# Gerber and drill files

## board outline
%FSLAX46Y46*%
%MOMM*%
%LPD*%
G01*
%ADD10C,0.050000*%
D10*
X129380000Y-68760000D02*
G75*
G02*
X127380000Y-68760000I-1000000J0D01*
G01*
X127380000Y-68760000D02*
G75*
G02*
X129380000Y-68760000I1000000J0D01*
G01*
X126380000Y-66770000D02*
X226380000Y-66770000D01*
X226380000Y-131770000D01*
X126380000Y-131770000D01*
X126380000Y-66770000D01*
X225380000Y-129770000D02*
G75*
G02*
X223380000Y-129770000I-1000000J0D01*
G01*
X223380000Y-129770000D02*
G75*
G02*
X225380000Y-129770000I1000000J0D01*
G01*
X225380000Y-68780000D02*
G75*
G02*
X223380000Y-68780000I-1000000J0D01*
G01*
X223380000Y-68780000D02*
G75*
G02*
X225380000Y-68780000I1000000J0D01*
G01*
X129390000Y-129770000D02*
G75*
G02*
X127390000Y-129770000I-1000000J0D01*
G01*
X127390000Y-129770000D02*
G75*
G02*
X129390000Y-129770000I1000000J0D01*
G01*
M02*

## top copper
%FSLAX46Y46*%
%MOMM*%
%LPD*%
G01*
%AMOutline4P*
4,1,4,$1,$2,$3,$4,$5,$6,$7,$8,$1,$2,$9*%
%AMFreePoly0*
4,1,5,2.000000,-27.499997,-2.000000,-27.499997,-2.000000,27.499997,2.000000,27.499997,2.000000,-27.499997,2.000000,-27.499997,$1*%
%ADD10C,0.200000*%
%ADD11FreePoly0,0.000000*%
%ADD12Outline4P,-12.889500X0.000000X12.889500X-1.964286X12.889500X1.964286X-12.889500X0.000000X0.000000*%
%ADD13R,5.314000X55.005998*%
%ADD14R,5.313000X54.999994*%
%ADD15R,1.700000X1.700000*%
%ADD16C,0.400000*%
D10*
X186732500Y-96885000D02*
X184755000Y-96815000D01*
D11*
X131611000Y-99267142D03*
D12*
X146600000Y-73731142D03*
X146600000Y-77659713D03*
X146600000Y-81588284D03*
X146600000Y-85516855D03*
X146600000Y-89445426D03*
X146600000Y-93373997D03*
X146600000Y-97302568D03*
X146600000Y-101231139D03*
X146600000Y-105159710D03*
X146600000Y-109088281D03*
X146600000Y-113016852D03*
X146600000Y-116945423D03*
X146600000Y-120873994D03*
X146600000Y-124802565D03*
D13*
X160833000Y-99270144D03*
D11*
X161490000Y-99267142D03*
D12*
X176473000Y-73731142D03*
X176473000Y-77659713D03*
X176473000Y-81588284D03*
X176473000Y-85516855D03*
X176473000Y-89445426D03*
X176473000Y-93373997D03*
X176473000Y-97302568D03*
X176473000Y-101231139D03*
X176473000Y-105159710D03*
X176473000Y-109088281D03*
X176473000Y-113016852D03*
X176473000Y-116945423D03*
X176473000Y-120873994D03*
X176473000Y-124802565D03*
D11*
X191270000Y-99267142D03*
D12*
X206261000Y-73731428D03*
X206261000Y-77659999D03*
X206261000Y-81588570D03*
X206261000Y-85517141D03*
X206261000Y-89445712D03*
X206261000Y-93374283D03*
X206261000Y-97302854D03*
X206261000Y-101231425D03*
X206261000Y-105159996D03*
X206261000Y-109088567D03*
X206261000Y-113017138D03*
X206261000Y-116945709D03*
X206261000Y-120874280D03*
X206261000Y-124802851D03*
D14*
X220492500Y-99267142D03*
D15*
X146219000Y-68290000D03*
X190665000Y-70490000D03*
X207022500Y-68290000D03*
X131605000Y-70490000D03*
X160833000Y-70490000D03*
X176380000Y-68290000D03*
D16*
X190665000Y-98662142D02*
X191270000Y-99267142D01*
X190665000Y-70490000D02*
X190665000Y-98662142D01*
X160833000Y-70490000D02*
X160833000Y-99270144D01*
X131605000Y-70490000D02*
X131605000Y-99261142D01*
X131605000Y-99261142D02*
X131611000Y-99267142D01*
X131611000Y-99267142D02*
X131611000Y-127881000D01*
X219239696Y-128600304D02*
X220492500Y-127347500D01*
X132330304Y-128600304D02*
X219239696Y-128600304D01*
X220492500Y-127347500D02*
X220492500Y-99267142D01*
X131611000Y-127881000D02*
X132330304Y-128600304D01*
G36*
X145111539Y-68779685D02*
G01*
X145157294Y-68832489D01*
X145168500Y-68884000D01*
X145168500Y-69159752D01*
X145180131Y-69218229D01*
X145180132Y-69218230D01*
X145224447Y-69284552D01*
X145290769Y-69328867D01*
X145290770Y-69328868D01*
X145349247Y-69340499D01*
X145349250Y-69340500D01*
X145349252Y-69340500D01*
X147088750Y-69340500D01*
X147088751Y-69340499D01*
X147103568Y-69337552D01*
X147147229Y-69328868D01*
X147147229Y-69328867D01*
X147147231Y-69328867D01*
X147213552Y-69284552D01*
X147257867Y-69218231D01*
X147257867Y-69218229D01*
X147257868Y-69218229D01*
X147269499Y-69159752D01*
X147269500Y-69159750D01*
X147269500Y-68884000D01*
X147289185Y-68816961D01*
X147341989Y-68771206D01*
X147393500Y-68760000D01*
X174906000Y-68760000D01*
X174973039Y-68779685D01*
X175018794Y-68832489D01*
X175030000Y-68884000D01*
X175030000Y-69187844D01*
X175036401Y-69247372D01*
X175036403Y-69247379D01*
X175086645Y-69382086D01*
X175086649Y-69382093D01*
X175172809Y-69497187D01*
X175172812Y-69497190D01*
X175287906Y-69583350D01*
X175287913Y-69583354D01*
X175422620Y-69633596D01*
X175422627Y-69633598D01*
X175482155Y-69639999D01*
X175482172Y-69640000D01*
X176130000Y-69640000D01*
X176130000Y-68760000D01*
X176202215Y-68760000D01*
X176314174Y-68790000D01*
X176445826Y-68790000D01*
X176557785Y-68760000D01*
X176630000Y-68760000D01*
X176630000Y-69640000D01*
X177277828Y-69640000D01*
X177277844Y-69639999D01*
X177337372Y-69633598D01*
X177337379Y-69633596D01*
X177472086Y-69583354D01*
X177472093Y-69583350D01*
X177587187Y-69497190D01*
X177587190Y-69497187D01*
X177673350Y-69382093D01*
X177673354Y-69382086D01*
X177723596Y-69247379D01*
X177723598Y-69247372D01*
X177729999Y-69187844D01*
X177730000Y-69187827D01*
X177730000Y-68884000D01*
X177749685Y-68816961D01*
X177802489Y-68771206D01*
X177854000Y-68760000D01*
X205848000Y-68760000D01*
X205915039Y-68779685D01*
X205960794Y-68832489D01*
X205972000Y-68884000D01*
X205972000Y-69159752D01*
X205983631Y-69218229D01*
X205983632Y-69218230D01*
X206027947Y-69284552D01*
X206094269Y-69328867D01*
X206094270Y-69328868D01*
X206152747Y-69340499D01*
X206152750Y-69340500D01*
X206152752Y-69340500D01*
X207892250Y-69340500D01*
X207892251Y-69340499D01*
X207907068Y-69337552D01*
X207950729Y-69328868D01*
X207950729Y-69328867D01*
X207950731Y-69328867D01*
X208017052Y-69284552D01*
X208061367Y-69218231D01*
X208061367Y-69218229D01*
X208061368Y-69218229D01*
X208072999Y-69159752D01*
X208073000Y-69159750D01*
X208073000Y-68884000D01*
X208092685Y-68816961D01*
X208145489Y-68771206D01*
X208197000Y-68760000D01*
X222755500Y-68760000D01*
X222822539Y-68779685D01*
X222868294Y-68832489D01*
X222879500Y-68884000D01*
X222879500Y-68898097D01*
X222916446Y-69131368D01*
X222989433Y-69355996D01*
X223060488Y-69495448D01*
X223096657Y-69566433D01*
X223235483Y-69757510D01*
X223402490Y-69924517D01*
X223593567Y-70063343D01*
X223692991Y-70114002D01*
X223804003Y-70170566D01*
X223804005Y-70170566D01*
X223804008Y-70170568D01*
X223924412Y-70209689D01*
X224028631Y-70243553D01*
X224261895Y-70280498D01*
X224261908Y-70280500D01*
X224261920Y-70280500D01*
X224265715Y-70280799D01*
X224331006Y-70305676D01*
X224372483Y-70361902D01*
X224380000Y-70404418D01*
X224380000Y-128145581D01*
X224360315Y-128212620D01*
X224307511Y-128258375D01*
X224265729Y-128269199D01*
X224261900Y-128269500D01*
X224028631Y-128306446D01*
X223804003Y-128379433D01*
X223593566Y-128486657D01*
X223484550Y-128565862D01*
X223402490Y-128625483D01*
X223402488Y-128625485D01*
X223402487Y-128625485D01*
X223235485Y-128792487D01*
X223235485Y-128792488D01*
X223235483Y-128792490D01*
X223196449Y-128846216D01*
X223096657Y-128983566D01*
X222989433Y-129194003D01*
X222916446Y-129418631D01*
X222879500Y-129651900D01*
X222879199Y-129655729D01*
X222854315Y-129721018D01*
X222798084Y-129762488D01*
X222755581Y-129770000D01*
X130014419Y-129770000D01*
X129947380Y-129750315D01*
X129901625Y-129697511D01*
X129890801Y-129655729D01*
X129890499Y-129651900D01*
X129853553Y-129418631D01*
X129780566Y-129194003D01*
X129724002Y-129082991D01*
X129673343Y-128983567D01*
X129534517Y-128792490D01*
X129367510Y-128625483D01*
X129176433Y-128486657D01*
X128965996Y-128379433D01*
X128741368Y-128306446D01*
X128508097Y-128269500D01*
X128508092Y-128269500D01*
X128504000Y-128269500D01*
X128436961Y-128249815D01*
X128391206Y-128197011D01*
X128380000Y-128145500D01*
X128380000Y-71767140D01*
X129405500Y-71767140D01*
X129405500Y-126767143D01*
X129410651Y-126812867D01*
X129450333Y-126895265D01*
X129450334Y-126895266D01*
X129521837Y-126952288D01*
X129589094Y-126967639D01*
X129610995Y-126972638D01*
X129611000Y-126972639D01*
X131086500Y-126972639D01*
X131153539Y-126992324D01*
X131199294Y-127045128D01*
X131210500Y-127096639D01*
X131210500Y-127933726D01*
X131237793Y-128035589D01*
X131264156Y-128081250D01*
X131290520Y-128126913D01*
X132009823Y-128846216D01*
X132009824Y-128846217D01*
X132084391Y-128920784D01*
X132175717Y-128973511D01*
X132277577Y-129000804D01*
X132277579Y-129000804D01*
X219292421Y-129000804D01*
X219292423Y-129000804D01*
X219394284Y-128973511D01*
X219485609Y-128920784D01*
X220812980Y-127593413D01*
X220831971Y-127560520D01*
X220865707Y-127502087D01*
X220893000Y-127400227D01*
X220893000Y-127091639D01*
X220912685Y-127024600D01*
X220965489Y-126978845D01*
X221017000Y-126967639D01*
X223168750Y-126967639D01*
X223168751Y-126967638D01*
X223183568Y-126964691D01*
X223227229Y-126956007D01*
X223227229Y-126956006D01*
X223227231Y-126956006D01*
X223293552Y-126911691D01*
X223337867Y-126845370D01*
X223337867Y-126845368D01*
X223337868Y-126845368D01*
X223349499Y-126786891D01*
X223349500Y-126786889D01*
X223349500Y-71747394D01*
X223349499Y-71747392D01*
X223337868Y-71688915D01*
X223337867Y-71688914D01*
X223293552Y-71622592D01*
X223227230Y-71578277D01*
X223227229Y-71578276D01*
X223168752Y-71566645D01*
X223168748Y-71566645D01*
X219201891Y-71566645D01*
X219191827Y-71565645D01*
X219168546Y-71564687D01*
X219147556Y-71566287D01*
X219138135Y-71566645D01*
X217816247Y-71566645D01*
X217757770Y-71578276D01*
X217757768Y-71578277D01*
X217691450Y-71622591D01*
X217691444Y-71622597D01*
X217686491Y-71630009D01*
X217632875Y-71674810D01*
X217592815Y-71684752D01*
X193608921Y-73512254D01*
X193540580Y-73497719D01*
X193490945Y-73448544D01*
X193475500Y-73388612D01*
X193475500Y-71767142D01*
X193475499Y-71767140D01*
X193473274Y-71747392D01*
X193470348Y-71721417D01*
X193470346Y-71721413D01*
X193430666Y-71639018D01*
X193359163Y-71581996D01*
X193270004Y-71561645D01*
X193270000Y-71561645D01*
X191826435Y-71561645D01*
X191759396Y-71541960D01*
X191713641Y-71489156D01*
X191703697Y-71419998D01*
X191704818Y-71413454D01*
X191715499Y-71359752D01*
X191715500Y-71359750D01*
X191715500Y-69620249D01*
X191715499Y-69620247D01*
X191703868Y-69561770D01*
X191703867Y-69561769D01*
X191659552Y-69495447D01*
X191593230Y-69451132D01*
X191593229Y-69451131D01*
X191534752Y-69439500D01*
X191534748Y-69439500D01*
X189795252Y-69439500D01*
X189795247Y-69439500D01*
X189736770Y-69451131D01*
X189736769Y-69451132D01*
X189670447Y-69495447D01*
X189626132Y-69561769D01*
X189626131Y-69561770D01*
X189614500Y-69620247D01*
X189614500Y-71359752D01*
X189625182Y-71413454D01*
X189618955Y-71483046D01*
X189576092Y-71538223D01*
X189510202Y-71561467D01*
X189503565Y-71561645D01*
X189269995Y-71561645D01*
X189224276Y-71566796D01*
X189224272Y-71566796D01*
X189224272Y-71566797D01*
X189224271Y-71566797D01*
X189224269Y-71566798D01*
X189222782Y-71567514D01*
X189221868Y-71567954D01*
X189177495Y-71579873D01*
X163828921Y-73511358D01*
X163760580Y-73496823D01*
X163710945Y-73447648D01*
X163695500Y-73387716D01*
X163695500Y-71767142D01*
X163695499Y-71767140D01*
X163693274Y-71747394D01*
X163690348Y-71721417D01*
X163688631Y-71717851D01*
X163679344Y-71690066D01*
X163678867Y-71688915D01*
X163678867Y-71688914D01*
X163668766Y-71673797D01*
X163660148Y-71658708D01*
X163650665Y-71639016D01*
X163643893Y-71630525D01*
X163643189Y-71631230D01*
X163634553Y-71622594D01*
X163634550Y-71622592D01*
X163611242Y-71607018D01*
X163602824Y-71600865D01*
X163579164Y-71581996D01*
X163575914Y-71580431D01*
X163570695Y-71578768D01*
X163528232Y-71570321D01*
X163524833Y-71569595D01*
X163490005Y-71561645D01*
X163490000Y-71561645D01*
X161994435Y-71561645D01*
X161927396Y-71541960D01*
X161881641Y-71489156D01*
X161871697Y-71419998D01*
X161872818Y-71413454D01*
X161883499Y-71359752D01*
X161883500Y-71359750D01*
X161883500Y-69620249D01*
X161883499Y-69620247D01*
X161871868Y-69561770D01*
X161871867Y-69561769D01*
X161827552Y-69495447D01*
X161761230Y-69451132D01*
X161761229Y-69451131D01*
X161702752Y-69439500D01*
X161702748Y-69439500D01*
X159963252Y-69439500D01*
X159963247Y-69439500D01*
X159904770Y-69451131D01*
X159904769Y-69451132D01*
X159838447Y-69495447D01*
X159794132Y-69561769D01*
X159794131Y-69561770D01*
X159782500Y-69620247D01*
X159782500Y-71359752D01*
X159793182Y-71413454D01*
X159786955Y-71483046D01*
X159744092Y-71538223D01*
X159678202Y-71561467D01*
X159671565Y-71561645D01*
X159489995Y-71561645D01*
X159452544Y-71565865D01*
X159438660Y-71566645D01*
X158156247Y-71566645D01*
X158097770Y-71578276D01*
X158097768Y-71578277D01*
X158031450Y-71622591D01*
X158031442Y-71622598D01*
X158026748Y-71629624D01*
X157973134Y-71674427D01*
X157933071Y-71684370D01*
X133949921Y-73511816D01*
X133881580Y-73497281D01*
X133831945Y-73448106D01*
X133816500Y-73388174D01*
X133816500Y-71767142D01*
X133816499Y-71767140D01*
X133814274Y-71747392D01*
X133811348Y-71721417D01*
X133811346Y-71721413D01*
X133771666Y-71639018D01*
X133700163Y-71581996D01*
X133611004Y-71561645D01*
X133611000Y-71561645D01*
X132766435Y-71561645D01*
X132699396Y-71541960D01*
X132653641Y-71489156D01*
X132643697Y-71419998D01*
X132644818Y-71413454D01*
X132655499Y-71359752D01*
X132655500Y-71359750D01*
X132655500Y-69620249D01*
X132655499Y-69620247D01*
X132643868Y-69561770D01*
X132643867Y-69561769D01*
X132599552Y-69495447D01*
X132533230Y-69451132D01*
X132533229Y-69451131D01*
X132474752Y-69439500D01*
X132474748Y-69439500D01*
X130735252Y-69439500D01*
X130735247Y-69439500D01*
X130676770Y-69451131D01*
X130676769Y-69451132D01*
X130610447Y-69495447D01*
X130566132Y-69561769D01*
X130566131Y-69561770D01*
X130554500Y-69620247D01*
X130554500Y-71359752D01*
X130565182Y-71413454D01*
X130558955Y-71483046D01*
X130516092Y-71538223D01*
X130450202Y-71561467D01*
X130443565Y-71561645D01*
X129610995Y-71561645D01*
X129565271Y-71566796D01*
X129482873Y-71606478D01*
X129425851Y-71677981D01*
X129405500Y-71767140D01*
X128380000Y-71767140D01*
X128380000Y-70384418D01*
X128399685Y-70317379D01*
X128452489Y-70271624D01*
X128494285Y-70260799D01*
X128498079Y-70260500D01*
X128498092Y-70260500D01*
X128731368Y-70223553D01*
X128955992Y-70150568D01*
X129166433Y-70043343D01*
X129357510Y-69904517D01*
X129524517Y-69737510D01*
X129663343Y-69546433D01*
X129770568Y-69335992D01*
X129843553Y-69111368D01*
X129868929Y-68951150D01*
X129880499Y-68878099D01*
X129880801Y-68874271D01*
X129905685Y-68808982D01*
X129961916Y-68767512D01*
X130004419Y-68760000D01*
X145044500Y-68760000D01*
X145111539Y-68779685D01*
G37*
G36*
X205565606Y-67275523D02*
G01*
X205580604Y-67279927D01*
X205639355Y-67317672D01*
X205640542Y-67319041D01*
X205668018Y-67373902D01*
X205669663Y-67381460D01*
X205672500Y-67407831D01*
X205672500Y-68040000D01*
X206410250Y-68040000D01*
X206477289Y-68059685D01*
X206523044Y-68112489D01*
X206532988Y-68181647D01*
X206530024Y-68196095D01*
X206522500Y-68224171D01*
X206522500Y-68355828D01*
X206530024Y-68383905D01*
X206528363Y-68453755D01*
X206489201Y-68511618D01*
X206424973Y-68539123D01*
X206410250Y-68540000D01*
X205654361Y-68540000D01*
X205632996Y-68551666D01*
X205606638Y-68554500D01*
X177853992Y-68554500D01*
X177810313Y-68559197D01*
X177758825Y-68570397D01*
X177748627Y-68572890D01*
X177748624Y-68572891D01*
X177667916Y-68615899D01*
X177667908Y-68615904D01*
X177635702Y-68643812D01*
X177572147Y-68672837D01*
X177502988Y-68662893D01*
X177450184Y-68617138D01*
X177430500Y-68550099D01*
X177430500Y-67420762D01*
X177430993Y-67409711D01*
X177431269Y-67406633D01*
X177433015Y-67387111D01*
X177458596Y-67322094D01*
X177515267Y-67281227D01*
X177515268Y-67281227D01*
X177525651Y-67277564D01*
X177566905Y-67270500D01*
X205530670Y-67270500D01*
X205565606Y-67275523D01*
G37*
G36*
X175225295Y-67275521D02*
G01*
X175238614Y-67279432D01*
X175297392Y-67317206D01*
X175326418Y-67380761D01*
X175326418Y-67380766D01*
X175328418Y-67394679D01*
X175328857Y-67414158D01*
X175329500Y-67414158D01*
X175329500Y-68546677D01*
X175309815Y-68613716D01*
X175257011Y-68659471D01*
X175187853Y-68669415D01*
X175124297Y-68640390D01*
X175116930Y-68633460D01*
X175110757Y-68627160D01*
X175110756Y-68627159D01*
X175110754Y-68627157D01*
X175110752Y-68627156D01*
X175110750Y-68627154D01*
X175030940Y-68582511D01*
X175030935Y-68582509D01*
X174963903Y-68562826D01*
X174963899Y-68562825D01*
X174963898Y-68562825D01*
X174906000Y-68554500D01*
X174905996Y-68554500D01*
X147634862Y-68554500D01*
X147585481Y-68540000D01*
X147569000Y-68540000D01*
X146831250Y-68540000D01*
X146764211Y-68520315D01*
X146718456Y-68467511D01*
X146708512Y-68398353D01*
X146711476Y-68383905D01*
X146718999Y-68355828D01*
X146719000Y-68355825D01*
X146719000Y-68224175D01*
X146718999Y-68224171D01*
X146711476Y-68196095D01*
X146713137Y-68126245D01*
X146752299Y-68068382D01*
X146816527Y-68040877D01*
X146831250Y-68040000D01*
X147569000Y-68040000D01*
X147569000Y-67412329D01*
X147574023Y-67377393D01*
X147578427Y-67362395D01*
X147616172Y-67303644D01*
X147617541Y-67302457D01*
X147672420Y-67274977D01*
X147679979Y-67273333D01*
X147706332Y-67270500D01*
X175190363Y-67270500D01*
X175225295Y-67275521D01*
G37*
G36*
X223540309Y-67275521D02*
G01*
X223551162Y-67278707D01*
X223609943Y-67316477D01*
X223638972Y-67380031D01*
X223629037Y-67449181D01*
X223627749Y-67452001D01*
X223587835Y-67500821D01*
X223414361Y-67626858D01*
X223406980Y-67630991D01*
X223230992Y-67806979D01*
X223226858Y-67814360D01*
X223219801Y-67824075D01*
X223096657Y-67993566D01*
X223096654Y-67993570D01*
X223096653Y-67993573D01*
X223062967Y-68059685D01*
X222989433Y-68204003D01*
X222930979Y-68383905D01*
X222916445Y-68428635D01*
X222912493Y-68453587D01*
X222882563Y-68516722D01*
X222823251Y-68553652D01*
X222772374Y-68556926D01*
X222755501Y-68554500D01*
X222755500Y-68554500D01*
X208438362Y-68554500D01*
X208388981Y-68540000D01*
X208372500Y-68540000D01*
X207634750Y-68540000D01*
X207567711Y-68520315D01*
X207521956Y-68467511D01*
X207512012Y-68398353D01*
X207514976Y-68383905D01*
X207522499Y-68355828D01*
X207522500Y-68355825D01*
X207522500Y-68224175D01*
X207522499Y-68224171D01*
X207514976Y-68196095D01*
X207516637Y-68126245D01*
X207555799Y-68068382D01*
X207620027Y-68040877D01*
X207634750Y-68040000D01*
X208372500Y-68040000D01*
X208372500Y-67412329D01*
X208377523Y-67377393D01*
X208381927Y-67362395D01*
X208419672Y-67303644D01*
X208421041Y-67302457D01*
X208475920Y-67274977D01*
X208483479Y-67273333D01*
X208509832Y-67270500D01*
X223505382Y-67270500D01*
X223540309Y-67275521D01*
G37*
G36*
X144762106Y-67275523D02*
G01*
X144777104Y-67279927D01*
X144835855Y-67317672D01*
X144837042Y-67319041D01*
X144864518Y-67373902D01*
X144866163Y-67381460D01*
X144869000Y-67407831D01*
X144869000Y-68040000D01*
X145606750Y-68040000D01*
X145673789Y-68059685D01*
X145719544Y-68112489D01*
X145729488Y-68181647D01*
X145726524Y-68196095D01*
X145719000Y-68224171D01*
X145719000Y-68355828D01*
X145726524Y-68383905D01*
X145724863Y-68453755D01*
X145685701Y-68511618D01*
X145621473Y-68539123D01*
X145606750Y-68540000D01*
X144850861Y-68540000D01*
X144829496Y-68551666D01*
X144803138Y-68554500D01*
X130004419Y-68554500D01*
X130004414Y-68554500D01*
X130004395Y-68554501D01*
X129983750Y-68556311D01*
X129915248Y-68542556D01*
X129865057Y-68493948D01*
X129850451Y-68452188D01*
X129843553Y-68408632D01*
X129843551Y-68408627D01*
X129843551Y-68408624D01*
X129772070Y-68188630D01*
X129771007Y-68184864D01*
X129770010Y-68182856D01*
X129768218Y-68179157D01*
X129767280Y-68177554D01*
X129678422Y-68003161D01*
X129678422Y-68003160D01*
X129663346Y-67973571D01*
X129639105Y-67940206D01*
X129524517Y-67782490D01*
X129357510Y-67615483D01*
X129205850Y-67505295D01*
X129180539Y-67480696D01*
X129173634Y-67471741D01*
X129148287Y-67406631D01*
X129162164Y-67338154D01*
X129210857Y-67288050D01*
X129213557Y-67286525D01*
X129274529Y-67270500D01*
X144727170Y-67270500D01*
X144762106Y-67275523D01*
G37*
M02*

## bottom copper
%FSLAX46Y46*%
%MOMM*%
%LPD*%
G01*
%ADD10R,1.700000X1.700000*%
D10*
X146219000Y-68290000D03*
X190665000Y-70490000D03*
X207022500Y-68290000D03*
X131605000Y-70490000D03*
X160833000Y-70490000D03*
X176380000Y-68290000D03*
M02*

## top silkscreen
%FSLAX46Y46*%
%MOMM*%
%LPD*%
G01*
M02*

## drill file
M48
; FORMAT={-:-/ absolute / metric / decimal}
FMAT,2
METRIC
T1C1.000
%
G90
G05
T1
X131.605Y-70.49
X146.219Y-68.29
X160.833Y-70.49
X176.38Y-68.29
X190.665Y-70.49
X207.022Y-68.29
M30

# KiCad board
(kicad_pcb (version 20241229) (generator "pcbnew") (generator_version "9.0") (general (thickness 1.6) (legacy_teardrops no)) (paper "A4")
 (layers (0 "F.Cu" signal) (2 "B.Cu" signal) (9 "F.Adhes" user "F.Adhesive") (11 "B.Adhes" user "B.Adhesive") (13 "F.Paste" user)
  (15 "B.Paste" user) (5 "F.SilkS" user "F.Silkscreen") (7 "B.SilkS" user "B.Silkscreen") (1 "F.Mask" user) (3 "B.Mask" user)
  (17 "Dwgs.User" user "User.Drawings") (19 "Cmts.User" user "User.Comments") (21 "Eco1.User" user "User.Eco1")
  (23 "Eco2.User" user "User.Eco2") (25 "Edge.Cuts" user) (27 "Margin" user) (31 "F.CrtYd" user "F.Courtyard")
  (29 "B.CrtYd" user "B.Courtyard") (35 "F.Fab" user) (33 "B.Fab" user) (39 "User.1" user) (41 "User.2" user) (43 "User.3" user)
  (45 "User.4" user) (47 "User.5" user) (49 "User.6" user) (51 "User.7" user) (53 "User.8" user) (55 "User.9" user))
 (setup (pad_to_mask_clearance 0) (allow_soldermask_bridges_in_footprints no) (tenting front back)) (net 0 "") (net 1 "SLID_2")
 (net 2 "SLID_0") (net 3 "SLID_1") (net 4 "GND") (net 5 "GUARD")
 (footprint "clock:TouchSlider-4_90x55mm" (layer "F.Cu") (at 176.332 99.267142)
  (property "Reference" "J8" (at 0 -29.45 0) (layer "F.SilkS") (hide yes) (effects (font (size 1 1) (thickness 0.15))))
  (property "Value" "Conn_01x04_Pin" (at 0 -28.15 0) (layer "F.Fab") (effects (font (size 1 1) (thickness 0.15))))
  (pad "1" smd custom (at -44.721 0) (size 4 54.999994) (layers "F.Cu") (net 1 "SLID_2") (thermal_bridge_angle 45)
   (options (clearance outline) (anchor rect)) (primitives))
  (pad "2" smd trapezoid (at -29.732 -25.536) (size 25.779 1.964285) (rect_delta -1.964285 0) (layers "F.Cu" "F.Paste") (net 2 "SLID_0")
   (thermal_bridge_angle 45))
  (pad "2" smd trapezoid (at -29.732 -21.607429) (size 25.779 1.964285) (rect_delta -1.964285 0) (layers "F.Cu" "F.Paste") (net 2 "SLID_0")
   (thermal_bridge_angle 45))
  (pad "2" smd trapezoid (at -29.732 -17.678858) (size 25.779 1.964285) (rect_delta -1.964285 0) (layers "F.Cu" "F.Paste") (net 2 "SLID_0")
   (thermal_bridge_angle 45))
  (pad "2" smd trapezoid (at -29.732 -13.750287) (size 25.779 1.964285) (rect_delta -1.964285 0) (layers "F.Cu" "F.Paste") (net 2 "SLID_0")
   (thermal_bridge_angle 45))
  (pad "2" smd trapezoid (at -29.732 -9.821716) (size 25.779 1.964285) (rect_delta -1.964285 0) (layers "F.Cu" "F.Paste") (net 2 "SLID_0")
   (thermal_bridge_angle 45))
  (pad "2" smd trapezoid (at -29.732 -5.893145) (size 25.779 1.964285) (rect_delta -1.964285 0) (layers "F.Cu" "F.Paste") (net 2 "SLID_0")
   (thermal_bridge_angle 45))
  (pad "2" smd trapezoid (at -29.732 -1.964574) (size 25.779 1.964285) (rect_delta -1.964285 0) (layers "F.Cu" "F.Paste") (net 2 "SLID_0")
   (thermal_bridge_angle 45))
  (pad "2" smd trapezoid (at -29.732 1.963997) (size 25.779 1.964285) (rect_delta -1.964285 0) (layers "F.Cu" "F.Paste") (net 2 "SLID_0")
   (thermal_bridge_angle 45))
  (pad "2" smd trapezoid (at -29.732 5.892568) (size 25.779 1.964285) (rect_delta -1.964285 0) (layers "F.Cu" "F.Paste") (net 2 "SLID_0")
   (thermal_bridge_angle 45))
  (pad "2" smd trapezoid (at -29.732 9.821139) (size 25.779 1.964285) (rect_delta -1.964285 0) (layers "F.Cu" "F.Paste") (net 2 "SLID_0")
   (thermal_bridge_angle 45))
  (pad "2" smd trapezoid (at -29.732 13.74971) (size 25.779 1.964285) (rect_delta -1.964285 0) (layers "F.Cu" "F.Paste") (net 2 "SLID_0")
   (thermal_bridge_angle 45))
  (pad "2" smd trapezoid (at -29.732 17.678281) (size 25.779 1.964285) (rect_delta -1.964285 0) (layers "F.Cu" "F.Paste") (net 2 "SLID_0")
   (thermal_bridge_angle 45))
  (pad "2" smd trapezoid (at -29.732 21.606852) (size 25.779 1.964285) (rect_delta -1.964285 0) (layers "F.Cu" "F.Paste") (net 2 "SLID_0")
   (thermal_bridge_angle 45))
  (pad "2" smd trapezoid (at -29.732 25.535423) (size 25.779 1.964285) (rect_delta -1.964285 0) (layers "F.Cu" "F.Paste") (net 2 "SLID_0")
   (thermal_bridge_angle 45))
  (pad "2" smd rect (at -15.499 0.003002) (size 5.314 55.005998) (layers "F.Cu") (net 2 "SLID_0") (thermal_bridge_angle 45))
  (pad "2" smd custom (at -14.842 0) (size 4 54.999994) (layers "F.Cu") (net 2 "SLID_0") (thermal_bridge_angle 45)
   (options (clearance outline) (anchor rect)) (primitives))
  (pad "3" smd trapezoid (at 0.141 -25.536) (size 25.779 1.964285) (rect_delta -1.964285 0) (layers "F.Cu" "F.Paste") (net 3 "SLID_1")
   (thermal_bridge_angle 45))
  (pad "3" smd trapezoid (at 0.141 -21.607429) (size 25.779 1.964285) (rect_delta -1.964285 0) (layers "F.Cu" "F.Paste") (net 3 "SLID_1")
   (thermal_bridge_angle 45))
  (pad "3" smd trapezoid (at 0.141 -17.678858) (size 25.779 1.964285) (rect_delta -1.964285 0) (layers "F.Cu" "F.Paste") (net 3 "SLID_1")
   (thermal_bridge_angle 45))
  (pad "3" smd trapezoid (at 0.141 -13.750287) (size 25.779 1.964285) (rect_delta -1.964285 0) (layers "F.Cu" "F.Paste") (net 3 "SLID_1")
   (thermal_bridge_angle 45))
  (pad "3" smd trapezoid (at 0.141 -9.821716) (size 25.779 1.964285) (rect_delta -1.964285 0) (layers "F.Cu" "F.Paste") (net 3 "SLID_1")
   (thermal_bridge_angle 45))
  (pad "3" smd trapezoid (at 0.141 -5.893145) (size 25.779 1.964285) (rect_delta -1.964285 0) (layers "F.Cu" "F.Paste") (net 3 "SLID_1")
   (thermal_bridge_angle 45))
  (pad "3" smd trapezoid (at 0.141 -1.964574) (size 25.779 1.964285) (rect_delta -1.964285 0) (layers "F.Cu" "F.Paste") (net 3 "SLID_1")
   (thermal_bridge_angle 45))
  (pad "3" smd trapezoid (at 0.141 1.963997) (size 25.779 1.964285) (rect_delta -1.964285 0) (layers "F.Cu" "F.Paste") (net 3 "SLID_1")
   (thermal_bridge_angle 45))
  (pad "3" smd trapezoid (at 0.141 5.892568) (size 25.779 1.964285) (rect_delta -1.964285 0) (layers "F.Cu" "F.Paste") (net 3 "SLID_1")
   (thermal_bridge_angle 45))
  (pad "3" smd trapezoid (at 0.141 9.821139) (size 25.779 1.964285) (rect_delta -1.964285 0) (layers "F.Cu" "F.Paste") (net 3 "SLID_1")
   (thermal_bridge_angle 45))
  (pad "3" smd trapezoid (at 0.141 13.74971) (size 25.779 1.964285) (rect_delta -1.964285 0) (layers "F.Cu" "F.Paste") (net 3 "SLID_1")
   (thermal_bridge_angle 45))
  (pad "3" smd trapezoid (at 0.141 17.678281) (size 25.779 1.964285) (rect_delta -1.964285 0) (layers "F.Cu" "F.Paste") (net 3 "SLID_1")
   (thermal_bridge_angle 45))
  (pad "3" smd trapezoid (at 0.141 21.606852) (size 25.779 1.964285) (rect_delta -1.964285 0) (layers "F.Cu" "F.Paste") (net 3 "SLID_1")
   (thermal_bridge_angle 45))
  (pad "3" smd trapezoid (at 0.141 25.535423) (size 25.779 1.964285) (rect_delta -1.964285 0) (layers "F.Cu" "F.Paste") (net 3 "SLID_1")
   (thermal_bridge_angle 45))
  (pad "3" smd custom (at 14.938 0) (size 4 54.999994) (layers "F.Cu") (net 3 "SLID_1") (thermal_bridge_angle 45)
   (options (clearance outline) (anchor rect)) (primitives))
  (pad "4" smd trapezoid (at 29.929 -25.535714) (size 25.779 1.964285) (rect_delta -1.964285 0) (layers "F.Cu" "F.Paste") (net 1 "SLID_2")
   (thermal_bridge_angle 45))
  (pad "4" smd trapezoid (at 29.929 -21.607143) (size 25.779 1.964285) (rect_delta -1.964285 0) (layers "F.Cu" "F.Paste") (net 1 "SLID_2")
   (thermal_bridge_angle 45))
  (pad "4" smd trapezoid (at 29.929 -17.678572) (size 25.779 1.964285) (rect_delta -1.964285 0) (layers "F.Cu" "F.Paste") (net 1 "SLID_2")
   (thermal_bridge_angle 45))
  (pad "4" smd trapezoid (at 29.929 -13.750001) (size 25.779 1.964285) (rect_delta -1.964285 0) (layers "F.Cu" "F.Paste") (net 1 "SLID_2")
   (thermal_bridge_angle 45))
  (pad "4" smd trapezoid (at 29.929 -9.82143) (size 25.779 1.964285) (rect_delta -1.964285 0) (layers "F.Cu" "F.Paste") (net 1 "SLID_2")
   (thermal_bridge_angle 45))
  (pad "4" smd trapezoid (at 29.929 -5.892859) (size 25.779 1.964285) (rect_delta -1.964285 0) (layers "F.Cu" "F.Paste") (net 1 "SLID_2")
   (thermal_bridge_angle 45))
  (pad "4" smd trapezoid (at 29.929 -1.964288) (size 25.779 1.964285) (rect_delta -1.964285 0) (layers "F.Cu" "F.Paste") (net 1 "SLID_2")
   (thermal_bridge_angle 45))
  (pad "4" smd trapezoid (at 29.929 1.964283) (size 25.779 1.964285) (rect_delta -1.964285 0) (layers "F.Cu" "F.Paste") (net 1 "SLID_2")
   (thermal_bridge_angle 45))
  (pad "4" smd trapezoid (at 29.929 5.892854) (size 25.779 1.964285) (rect_delta -1.964285 0) (layers "F.Cu" "F.Paste") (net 1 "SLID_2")
   (thermal_bridge_angle 45))
  (pad "4" smd trapezoid (at 29.929 9.821425) (size 25.779 1.964285) (rect_delta -1.964285 0) (layers "F.Cu" "F.Paste") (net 1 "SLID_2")
   (thermal_bridge_angle 45))
  (pad "4" smd trapezoid (at 29.929 13.749996) (size 25.779 1.964285) (rect_delta -1.964285 0) (layers "F.Cu" "F.Paste") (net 1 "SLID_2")
   (thermal_bridge_angle 45))
  (pad "4" smd trapezoid (at 29.929 17.678567) (size 25.779 1.964285) (rect_delta -1.964285 0) (layers "F.Cu" "F.Paste") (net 1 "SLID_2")
   (thermal_bridge_angle 45))
  (pad "4" smd trapezoid (at 29.929 21.607138) (size 25.779 1.964285) (rect_delta -1.964285 0) (layers "F.Cu" "F.Paste") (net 1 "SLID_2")
   (thermal_bridge_angle 45))
  (pad "4" smd trapezoid (at 29.929 25.535709) (size 25.779 1.964285) (rect_delta -1.964285 0) (layers "F.Cu" "F.Paste") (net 1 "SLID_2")
   (thermal_bridge_angle 45))
  (pad "4" smd rect (at 44.1605 0) (size 5.313 54.999994) (layers "F.Cu") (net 1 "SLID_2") (thermal_bridge_angle 45)))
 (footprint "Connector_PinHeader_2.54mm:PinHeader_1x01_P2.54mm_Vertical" (layer "B.Cu") (at 146.219 68.29 90)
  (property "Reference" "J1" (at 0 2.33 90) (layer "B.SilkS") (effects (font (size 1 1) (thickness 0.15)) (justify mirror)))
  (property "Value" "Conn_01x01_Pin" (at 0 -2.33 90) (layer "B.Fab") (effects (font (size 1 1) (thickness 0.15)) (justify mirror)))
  (pad "1" thru_hole rect (at 0 0 90) (size 1.7 1.7) (drill 1) (layers "*.Cu" "*.Mask") (remove_unused_layers no) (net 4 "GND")))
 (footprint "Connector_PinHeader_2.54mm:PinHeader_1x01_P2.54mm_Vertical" (layer "B.Cu") (at 190.665 70.49 180)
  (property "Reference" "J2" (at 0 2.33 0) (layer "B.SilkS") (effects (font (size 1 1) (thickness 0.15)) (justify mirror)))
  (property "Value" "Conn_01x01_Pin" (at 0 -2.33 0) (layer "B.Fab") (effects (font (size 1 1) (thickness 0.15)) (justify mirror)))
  (pad "1" thru_hole rect (at 0 0 180) (size 1.7 1.7) (drill 1) (layers "*.Cu" "*.Mask") (remove_unused_layers no) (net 3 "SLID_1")))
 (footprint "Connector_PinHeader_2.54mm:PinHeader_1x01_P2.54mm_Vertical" (layer "B.Cu") (at 207.0225 68.29 180)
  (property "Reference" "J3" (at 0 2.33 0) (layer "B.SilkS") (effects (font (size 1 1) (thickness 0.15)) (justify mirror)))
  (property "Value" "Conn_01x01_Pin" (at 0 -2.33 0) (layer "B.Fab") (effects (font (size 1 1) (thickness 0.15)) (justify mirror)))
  (pad "1" thru_hole rect (at 0 0 180) (size 1.7 1.7) (drill 1) (layers "*.Cu" "*.Mask") (remove_unused_layers no) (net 4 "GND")))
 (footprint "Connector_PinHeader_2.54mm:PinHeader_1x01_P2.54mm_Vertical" (layer "B.Cu") (at 131.605 70.49 180)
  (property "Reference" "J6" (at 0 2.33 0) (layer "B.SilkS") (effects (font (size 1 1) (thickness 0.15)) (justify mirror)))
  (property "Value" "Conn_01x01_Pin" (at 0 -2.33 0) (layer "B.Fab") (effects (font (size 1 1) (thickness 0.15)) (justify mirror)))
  (pad "1" thru_hole rect (at 0 0 180) (size 1.7 1.7) (drill 1) (layers "*.Cu" "*.Mask") (remove_unused_layers no) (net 1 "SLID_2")))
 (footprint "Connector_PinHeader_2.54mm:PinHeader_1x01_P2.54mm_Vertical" (layer "B.Cu") (at 160.833 70.49 180)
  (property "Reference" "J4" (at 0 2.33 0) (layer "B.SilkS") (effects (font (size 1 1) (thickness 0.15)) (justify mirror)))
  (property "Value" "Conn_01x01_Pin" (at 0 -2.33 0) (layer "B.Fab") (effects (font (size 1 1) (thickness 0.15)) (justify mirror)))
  (pad "1" thru_hole rect (at 0 0 180) (size 1.7 1.7) (drill 1) (layers "*.Cu" "*.Mask") (remove_unused_layers no) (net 2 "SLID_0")))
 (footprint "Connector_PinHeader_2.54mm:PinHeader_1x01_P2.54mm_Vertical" (layer "B.Cu") (at 176.38 68.29 180)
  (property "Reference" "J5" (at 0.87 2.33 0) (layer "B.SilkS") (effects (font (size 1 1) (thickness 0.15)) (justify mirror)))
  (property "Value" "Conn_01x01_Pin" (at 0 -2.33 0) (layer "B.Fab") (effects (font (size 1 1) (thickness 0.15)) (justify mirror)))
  (pad "1" thru_hole rect (at 0 0 180) (size 1.7 1.7) (drill 1) (layers "*.Cu" "*.Mask") (remove_unused_layers no) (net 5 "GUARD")))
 (gr_line (start 186.7325 96.885) (end 184.755 96.815) (stroke (width 0.2) (type default)) (layer "F.Cu") (net 3))
 (gr_circle (center 128.38 68.76) (end 129.38 68.76) (stroke (width 0.05) (type default)) (fill no) (layer "Edge.Cuts"))
 (gr_rect (start 126.38 66.77) (end 226.38 131.77) (stroke (width 0.05) (type solid)) (fill no) (locked yes) (layer "Edge.Cuts"))
 (gr_circle (center 224.38 129.77) (end 223.38 129.77) (stroke (width 0.05) (type default)) (fill no) (layer "Edge.Cuts"))
 (gr_circle (center 224.38 68.78) (end 224.38 69.78) (stroke (width 0.05) (type default)) (fill no) (layer "Edge.Cuts"))
 (gr_circle (center 128.39 129.77) (end 128.39 128.77) (stroke (width 0.05) (type default)) (fill no) (layer "Edge.Cuts"))
 (segment (start 190.665 98.662142) (end 191.27 99.267142) (width 0.4) (layer "F.Cu") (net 3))
 (segment (start 190.665 70.49) (end 190.665 98.662142) (width 0.4) (layer "F.Cu") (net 3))
 (segment (start 160.833 70.49) (end 160.833 99.270144) (width 0.4) (layer "F.Cu") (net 2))
 (segment (start 131.605 70.49) (end 131.605 99.261142) (width 0.4) (layer "F.Cu") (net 1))
 (segment (start 131.605 99.261142) (end 131.611 99.267142) (width 0.4) (layer "F.Cu") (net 1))
 (segment (start 131.611 99.267142) (end 131.611 127.881) (width 0.4) (layer "F.Cu") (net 1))
 (segment (start 219.239696 128.600304) (end 220.4925 127.3475) (width 0.4) (layer "F.Cu") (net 1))
 (segment (start 132.330304 128.600304) (end 219.239696 128.600304) (width 0.4) (layer "F.Cu") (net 1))
 (segment (start 220.4925 127.3475) (end 220.4925 99.267142) (width 0.4) (layer "F.Cu") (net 1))
 (segment (start 131.611 127.881) (end 132.330304 128.600304) (width 0.4) (layer "F.Cu") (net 1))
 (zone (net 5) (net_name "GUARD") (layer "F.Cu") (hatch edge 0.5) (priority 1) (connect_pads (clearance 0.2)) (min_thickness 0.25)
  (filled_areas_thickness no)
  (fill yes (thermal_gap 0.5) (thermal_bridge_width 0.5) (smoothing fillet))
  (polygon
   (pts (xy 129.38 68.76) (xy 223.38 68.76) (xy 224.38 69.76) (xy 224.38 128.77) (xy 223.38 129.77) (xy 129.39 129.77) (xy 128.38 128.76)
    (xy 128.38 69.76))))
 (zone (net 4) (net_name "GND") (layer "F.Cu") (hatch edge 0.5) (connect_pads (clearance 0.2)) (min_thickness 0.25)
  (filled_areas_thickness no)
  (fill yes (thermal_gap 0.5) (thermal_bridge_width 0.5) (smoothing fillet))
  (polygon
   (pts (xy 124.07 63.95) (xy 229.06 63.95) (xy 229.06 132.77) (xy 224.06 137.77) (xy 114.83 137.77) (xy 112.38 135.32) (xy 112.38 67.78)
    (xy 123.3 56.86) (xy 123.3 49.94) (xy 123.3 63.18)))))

